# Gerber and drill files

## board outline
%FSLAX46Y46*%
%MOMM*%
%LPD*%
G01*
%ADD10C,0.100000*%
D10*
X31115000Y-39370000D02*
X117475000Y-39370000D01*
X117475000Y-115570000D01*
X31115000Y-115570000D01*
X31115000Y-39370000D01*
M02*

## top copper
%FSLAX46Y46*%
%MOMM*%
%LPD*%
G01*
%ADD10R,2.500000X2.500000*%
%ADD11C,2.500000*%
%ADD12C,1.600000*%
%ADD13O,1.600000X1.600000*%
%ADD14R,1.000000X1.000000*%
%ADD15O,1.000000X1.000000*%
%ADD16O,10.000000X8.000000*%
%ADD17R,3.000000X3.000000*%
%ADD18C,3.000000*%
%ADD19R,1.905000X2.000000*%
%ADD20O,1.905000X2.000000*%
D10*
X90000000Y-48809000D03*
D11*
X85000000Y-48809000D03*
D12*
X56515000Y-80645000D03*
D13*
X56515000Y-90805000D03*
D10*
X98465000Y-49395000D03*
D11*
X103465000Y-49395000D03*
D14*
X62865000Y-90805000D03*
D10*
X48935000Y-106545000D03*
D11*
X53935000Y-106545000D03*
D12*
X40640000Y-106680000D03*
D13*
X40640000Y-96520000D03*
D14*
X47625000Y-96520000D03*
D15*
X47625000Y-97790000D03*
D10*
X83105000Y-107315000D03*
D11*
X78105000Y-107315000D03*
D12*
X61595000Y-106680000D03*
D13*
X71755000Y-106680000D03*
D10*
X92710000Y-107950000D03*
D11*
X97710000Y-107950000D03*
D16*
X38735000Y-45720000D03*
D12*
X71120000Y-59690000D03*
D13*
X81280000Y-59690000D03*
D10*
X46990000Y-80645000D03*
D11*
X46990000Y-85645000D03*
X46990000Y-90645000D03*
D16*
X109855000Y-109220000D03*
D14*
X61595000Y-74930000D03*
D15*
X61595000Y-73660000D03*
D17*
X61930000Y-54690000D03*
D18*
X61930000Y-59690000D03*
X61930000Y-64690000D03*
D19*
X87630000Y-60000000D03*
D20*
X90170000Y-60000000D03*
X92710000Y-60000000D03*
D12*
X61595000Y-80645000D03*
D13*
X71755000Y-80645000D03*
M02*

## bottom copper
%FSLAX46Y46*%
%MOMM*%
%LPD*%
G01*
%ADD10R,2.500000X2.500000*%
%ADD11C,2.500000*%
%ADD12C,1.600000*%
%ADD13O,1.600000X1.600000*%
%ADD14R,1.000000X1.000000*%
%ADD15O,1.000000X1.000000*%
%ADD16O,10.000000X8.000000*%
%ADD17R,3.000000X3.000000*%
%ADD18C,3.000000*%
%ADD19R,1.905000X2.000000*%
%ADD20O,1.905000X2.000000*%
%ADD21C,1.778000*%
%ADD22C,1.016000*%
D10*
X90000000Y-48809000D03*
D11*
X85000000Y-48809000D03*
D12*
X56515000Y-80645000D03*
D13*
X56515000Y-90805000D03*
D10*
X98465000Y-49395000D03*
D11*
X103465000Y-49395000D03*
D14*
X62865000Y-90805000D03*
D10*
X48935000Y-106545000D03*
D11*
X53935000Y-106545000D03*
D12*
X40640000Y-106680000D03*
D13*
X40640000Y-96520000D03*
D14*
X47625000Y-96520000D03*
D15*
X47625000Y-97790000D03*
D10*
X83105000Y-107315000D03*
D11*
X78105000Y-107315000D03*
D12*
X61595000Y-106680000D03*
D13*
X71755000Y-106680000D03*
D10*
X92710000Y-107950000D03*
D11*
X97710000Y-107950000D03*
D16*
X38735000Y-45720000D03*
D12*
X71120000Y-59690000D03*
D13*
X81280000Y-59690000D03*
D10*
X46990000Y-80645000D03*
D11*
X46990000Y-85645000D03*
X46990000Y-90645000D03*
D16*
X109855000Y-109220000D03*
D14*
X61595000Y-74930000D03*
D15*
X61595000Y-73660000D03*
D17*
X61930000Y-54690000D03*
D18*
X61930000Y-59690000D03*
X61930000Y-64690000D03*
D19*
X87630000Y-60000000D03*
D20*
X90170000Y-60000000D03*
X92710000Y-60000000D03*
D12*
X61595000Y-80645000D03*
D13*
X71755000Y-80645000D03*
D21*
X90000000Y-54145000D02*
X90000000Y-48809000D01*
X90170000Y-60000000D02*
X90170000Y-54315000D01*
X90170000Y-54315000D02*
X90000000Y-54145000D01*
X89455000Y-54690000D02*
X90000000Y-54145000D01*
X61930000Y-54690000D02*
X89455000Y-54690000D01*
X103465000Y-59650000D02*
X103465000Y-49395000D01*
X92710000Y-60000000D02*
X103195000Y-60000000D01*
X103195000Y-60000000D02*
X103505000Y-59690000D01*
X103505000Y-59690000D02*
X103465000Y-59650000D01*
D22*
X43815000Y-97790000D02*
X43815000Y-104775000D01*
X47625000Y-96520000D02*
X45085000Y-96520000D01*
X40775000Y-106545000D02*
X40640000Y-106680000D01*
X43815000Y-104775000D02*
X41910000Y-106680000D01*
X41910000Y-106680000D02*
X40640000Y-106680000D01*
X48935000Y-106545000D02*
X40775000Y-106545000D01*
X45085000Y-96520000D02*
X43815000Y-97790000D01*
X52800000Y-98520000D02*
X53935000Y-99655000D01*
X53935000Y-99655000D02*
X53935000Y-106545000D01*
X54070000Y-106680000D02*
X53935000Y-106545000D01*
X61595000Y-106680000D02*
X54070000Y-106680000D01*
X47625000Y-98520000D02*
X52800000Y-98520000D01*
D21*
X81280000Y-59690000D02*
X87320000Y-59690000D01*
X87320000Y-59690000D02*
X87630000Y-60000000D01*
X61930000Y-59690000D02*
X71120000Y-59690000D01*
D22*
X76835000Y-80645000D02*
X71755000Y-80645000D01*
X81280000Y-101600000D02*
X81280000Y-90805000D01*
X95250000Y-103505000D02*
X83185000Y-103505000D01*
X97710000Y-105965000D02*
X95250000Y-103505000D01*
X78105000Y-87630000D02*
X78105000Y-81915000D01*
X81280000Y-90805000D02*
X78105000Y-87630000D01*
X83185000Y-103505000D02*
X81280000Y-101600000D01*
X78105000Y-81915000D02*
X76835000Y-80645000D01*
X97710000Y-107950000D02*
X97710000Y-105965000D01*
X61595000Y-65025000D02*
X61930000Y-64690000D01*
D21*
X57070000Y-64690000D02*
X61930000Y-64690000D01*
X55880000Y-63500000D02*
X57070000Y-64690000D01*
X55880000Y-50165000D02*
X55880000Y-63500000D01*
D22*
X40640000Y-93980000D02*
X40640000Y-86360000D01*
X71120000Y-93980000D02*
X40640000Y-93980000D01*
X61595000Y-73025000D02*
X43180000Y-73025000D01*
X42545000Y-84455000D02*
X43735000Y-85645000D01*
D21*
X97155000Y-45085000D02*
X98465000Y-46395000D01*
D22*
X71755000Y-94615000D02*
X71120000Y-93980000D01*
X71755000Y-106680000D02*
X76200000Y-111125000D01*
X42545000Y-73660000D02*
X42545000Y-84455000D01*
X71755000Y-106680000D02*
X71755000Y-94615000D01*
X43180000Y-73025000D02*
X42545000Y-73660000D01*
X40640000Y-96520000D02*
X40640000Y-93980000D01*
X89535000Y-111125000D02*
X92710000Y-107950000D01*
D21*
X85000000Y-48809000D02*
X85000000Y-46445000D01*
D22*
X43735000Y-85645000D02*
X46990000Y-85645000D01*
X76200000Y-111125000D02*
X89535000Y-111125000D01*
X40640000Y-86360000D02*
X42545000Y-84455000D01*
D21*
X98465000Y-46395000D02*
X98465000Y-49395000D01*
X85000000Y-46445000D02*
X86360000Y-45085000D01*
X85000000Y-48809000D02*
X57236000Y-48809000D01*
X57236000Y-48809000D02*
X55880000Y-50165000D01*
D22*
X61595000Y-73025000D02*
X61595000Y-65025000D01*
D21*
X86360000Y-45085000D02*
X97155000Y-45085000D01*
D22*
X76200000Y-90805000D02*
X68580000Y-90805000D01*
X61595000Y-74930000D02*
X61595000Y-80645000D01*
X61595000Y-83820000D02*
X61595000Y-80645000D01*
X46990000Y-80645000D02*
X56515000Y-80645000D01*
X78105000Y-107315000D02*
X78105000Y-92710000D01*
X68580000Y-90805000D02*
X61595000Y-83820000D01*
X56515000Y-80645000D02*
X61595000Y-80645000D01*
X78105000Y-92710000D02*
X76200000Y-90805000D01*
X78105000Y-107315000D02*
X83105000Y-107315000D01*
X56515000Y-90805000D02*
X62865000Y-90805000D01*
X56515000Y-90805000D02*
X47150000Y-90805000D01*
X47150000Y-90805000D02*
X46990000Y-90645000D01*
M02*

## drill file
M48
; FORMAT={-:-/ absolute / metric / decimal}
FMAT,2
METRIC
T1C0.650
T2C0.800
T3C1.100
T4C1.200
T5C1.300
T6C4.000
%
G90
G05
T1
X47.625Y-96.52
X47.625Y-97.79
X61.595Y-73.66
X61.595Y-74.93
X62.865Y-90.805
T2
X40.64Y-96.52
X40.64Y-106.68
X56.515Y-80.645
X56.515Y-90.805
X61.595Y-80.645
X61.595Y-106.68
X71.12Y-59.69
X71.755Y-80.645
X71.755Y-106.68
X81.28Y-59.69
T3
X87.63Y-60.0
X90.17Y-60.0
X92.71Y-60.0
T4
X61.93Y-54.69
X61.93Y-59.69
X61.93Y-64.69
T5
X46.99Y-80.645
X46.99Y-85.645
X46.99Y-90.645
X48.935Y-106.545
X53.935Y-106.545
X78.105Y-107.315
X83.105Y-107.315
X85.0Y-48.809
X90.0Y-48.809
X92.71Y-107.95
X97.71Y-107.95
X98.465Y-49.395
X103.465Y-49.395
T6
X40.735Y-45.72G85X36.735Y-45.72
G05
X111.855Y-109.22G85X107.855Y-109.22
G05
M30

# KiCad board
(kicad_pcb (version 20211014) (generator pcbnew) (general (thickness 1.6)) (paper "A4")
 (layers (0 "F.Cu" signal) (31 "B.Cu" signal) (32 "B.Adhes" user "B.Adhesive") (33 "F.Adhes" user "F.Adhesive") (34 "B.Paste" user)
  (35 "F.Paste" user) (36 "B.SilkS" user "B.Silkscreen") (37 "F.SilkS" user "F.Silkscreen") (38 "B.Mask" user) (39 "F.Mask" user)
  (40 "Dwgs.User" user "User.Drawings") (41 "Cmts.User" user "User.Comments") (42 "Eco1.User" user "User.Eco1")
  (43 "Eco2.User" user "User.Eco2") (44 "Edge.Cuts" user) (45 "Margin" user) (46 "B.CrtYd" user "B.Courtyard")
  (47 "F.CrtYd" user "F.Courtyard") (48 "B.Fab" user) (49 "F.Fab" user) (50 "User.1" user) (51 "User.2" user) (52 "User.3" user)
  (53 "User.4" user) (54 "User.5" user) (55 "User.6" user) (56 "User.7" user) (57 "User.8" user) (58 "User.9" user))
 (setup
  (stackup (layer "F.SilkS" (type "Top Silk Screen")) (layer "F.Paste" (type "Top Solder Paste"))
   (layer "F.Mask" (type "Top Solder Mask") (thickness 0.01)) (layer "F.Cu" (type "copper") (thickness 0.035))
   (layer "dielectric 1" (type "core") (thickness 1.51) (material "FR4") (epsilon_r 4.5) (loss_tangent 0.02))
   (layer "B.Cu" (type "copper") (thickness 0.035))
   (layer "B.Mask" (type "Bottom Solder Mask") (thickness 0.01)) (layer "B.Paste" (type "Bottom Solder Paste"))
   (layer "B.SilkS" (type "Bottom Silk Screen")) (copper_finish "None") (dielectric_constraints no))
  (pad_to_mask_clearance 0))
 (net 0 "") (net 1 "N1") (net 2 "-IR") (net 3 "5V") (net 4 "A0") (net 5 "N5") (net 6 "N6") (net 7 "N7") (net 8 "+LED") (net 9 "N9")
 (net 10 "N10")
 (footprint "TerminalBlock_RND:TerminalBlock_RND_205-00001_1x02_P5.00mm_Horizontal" (layer "F.Cu") (at 90 48.809 180)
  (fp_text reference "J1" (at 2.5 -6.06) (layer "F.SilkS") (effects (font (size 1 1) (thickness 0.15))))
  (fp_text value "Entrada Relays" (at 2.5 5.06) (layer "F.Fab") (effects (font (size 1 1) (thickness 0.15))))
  (pad "1" thru_hole rect (at 0 0 180) (size 2.5 2.5) (drill 1.3) (layers *.Cu *.Mask) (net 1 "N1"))
  (pad "2" thru_hole circle (at 5 0 180) (size 2.5 2.5) (drill 1.3) (layers *.Cu *.Mask) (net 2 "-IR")))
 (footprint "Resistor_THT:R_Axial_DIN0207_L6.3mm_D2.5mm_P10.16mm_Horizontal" (layer "F.Cu") (at 56.515 80.645 -90)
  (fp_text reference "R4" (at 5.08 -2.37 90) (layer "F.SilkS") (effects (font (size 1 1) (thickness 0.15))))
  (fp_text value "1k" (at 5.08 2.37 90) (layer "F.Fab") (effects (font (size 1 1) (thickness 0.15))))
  (pad "1" thru_hole circle (at 0 0 270) (size 1.6 1.6) (drill 0.8) (layers *.Cu *.Mask) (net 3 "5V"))
  (pad "2" thru_hole oval (at 10.16 0 270) (size 1.6 1.6) (drill 0.8) (layers *.Cu *.Mask) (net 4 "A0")))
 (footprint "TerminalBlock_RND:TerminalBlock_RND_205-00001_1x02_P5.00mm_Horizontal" (layer "F.Cu") (at 98.465 49.395)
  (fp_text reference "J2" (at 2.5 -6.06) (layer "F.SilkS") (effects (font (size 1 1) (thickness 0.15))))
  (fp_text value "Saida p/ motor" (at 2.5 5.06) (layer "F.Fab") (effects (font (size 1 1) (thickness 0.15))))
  (pad "1" thru_hole rect (at 0 0) (size 2.5 2.5) (drill 1.3) (layers *.Cu *.Mask) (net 2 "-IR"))
  (pad "2" thru_hole circle (at 5 0) (size 2.5 2.5) (drill 1.3) (layers *.Cu *.Mask) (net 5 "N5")))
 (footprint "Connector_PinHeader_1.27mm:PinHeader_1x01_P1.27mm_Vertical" (layer "F.Cu") (at 62.865 90.805)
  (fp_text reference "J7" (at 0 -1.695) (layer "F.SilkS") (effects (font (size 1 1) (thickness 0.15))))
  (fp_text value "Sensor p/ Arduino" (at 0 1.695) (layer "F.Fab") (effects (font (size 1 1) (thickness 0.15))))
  (pad "1" thru_hole rect (at 0 0) (size 1 1) (drill 0.65) (layers *.Cu *.Mask) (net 4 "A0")))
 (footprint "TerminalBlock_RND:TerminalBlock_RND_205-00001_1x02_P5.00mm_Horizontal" (layer "F.Cu") (at 48.935 106.545)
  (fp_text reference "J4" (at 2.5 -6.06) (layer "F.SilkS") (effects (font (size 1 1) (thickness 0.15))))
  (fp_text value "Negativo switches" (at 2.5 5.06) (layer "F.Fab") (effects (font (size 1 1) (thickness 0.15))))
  (pad "1" thru_hole rect (at 0 0) (size 2.5 2.5) (drill 1.3) (layers *.Cu *.Mask) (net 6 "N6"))
  (pad "2" thru_hole circle (at 5 0) (size 2.5 2.5) (drill 1.3) (layers *.Cu *.Mask) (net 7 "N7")))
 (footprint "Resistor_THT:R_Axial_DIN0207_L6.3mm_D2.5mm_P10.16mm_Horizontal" (layer "F.Cu") (at 40.64 106.68 90)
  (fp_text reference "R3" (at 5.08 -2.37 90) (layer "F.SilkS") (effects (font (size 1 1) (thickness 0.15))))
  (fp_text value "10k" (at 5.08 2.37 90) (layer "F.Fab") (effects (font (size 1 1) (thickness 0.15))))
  (pad "1" thru_hole circle (at 0 0 90) (size 1.6 1.6) (drill 0.8) (layers *.Cu *.Mask) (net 6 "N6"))
  (pad "2" thru_hole oval (at 10.16 0 90) (size 1.6 1.6) (drill 0.8) (layers *.Cu *.Mask) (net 2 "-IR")))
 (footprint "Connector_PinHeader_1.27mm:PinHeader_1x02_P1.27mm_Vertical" (layer "F.Cu") (at 47.625 96.52)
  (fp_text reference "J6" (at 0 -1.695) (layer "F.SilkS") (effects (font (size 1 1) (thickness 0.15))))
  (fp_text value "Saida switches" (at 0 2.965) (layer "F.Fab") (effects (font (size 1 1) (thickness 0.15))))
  (pad "1" thru_hole rect (at 0 0) (size 1 1) (drill 0.65) (layers *.Cu *.Mask) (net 6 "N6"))
  (pad "2" thru_hole oval (at 0 1.27) (size 1 1) (drill 0.65) (layers *.Cu *.Mask) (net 7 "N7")))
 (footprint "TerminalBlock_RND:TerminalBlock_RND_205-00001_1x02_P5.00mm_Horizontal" (layer "F.Cu") (at 83.105 107.315 180)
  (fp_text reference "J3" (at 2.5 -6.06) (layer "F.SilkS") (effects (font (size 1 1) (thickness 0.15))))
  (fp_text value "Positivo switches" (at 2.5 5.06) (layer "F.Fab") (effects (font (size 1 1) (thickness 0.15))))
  (pad "1" thru_hole rect (at 0 0 180) (size 2.5 2.5) (drill 1.3) (layers *.Cu *.Mask) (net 3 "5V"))
  (pad "2" thru_hole circle (at 5 0 180) (size 2.5 2.5) (drill 1.3) (layers *.Cu *.Mask) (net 3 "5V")))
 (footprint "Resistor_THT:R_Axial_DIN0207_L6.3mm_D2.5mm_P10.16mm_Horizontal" (layer "F.Cu") (at 61.595 106.68)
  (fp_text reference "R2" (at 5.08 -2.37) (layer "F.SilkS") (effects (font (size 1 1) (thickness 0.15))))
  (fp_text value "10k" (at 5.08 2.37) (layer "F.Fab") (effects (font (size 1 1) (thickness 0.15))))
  (pad "1" thru_hole circle (at 0 0) (size 1.6 1.6) (drill 0.8) (layers *.Cu *.Mask) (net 7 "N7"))
  (pad "2" thru_hole oval (at 10.16 0) (size 1.6 1.6) (drill 0.8) (layers *.Cu *.Mask) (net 2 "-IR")))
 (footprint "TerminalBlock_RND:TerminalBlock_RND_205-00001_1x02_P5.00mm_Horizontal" (layer "F.Cu") (at 92.71 107.95)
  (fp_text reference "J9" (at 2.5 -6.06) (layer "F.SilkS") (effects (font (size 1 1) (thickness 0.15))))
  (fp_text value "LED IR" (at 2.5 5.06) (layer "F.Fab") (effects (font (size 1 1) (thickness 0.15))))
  (pad "1" thru_hole rect (at 0 0) (size 2.5 2.5) (drill 1.3) (layers *.Cu *.Mask) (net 2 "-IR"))
  (pad "2" thru_hole circle (at 5 0) (size 2.5 2.5) (drill 1.3) (layers *.Cu *.Mask) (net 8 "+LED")))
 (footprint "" (layer "F.Cu") (at 38.735 45.72)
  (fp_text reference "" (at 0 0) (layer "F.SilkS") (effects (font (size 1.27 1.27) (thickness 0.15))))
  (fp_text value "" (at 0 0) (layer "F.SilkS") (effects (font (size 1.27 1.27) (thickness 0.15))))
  (pad "1" thru_hole oval (at 0 0 180) (size 10 8) (drill oval 8 4) (layers *.Cu *.Mask)))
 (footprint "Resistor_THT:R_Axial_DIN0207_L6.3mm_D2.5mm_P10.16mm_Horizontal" (layer "F.Cu") (at 71.12 59.69)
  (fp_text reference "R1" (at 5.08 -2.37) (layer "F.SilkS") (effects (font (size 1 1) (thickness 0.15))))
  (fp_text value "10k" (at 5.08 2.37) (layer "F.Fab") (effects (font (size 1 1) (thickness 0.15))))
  (pad "1" thru_hole circle (at 0 0) (size 1.6 1.6) (drill 0.8) (layers *.Cu *.Mask) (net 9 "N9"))
  (pad "2" thru_hole oval (at 10.16 0) (size 1.6 1.6) (drill 0.8) (layers *.Cu *.Mask) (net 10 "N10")))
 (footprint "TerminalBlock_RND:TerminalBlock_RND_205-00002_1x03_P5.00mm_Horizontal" (layer "F.Cu") (at 46.99 80.645 -90)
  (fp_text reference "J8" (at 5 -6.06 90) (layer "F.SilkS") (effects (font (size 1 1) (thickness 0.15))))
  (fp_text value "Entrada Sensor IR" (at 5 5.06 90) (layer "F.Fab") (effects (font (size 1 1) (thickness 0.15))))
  (pad "1" thru_hole rect (at 0 0 270) (size 2.5 2.5) (drill 1.3) (layers *.Cu *.Mask) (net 3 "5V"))
  (pad "2" thru_hole circle (at 5 0 270) (size 2.5 2.5) (drill 1.3) (layers *.Cu *.Mask) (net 2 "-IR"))
  (pad "3" thru_hole circle (at 10 0 270) (size 2.5 2.5) (drill 1.3) (layers *.Cu *.Mask) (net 4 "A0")))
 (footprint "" (layer "F.Cu") (at 109.855 109.22)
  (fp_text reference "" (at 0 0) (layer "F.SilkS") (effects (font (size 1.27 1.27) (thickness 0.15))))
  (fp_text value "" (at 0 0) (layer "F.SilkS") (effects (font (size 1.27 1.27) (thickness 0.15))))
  (pad "1" thru_hole oval (at 0 0 180) (size 10 8) (drill oval 8 4) (layers F&B.Cu *.Mask)))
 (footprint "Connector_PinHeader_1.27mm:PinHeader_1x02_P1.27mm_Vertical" (layer "F.Cu") (at 61.595 74.93 180)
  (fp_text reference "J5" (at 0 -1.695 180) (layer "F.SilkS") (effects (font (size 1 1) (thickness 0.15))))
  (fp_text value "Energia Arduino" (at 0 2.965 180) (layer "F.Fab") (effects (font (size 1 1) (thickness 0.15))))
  (pad "1" thru_hole rect (at 0 0 180) (size 1 1) (drill 0.65) (layers *.Cu *.Mask) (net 3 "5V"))
  (pad "2" thru_hole oval (at 0 1.27 180) (size 1 1) (drill 0.65) (layers *.Cu *.Mask) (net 2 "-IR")))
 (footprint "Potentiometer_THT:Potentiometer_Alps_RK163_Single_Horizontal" (layer "F.Cu") (at 61.93 54.69)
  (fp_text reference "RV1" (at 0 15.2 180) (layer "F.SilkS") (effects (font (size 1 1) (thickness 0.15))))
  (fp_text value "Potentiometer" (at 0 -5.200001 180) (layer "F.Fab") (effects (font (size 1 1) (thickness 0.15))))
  (pad "1" thru_hole rect (at 0 0 180) (size 3 3) (drill 1.2) (layers *.Cu *.Mask) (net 1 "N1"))
  (pad "2" thru_hole circle (at 0 5 180) (size 3 3) (drill 1.2) (layers *.Cu *.Mask) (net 9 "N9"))
  (pad "3" thru_hole circle (at 0 10 180) (size 3 3) (drill 1.2) (layers *.Cu *.Mask) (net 2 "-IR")))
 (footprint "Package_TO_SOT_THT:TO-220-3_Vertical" (layer "F.Cu") (at 87.63 60)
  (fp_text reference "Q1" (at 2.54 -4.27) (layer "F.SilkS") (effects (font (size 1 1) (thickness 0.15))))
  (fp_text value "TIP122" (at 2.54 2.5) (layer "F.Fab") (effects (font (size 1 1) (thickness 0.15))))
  (pad "1" thru_hole rect (at 0 0) (size 1.905 2) (drill 1.1) (layers *.Cu *.Mask) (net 10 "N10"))
  (pad "2" thru_hole oval (at 2.54 0) (size 1.905 2) (drill 1.1) (layers *.Cu *.Mask) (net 1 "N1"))
  (pad "3" thru_hole oval (at 5.08 0) (size 1.905 2) (drill 1.1) (layers *.Cu *.Mask) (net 5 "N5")))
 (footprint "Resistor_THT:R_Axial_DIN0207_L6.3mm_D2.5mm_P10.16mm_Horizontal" (layer "F.Cu") (at 61.595 80.645)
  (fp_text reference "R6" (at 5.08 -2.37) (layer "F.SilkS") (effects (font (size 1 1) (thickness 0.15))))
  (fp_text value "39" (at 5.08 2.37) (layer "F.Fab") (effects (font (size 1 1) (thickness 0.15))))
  (pad "1" thru_hole circle (at 0 0) (size 1.6 1.6) (drill 0.8) (layers *.Cu *.Mask) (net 3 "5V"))
  (pad "2" thru_hole oval (at 10.16 0) (size 1.6 1.6) (drill 0.8) (layers *.Cu *.Mask) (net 8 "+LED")))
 (gr_rect (start 117.475 39.37) (end 31.115 115.57) (layer "Edge.Cuts") (width 0.1) (fill none))
 (segment (start 90 54.145) (end 90 48.809) (width 1.778) (layer "B.Cu") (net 1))
 (segment (start 90.17 60) (end 90.17 54.315) (width 1.778) (layer "B.Cu") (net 1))
 (segment (start 90.17 54.315) (end 90 54.145) (width 1.778) (layer "B.Cu") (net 1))
 (segment (start 89.455 54.69) (end 90 54.145) (width 1.778) (layer "B.Cu") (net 1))
 (segment (start 61.93 54.69) (end 89.455 54.69) (width 1.778) (layer "B.Cu") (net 1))
 (segment (start 103.465 59.65) (end 103.465 49.395) (width 1.778) (layer "B.Cu") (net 5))
 (segment (start 92.71 60) (end 103.195 60) (width 1.778) (layer "B.Cu") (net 5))
 (segment (start 103.195 60) (end 103.505 59.69) (width 1.778) (layer "B.Cu") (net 5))
 (segment (start 103.505 59.69) (end 103.465 59.65) (width 1.778) (layer "B.Cu") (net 5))
 (segment (start 43.815 97.79) (end 43.815 104.775) (width 1.016) (layer "B.Cu") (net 6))
 (segment (start 47.625 96.52) (end 45.085 96.52) (width 1.016) (layer "B.Cu") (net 6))
 (segment (start 40.775 106.545) (end 40.64 106.68) (width 1.016) (layer "B.Cu") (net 6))
 (segment (start 43.815 104.775) (end 41.91 106.68) (width 1.016) (layer "B.Cu") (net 6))
 (segment (start 41.91 106.68) (end 40.64 106.68) (width 1.016) (layer "B.Cu") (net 6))
 (segment (start 48.935 106.545) (end 40.775 106.545) (width 1.016) (layer "B.Cu") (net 6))
 (segment (start 45.085 96.52) (end 43.815 97.79) (width 1.016) (layer "B.Cu") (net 6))
 (segment (start 52.8 98.52) (end 53.935 99.655) (width 1.016) (layer "B.Cu") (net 7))
 (segment (start 53.935 99.655) (end 53.935 106.545) (width 1.016) (layer "B.Cu") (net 7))
 (segment (start 54.07 106.68) (end 53.935 106.545) (width 1.016) (layer "B.Cu") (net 7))
 (segment (start 61.595 106.68) (end 54.07 106.68) (width 1.016) (layer "B.Cu") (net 7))
 (segment (start 47.625 98.52) (end 52.8 98.52) (width 1.016) (layer "B.Cu") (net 7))
 (segment (start 81.28 59.69) (end 87.32 59.69) (width 1.778) (layer "B.Cu") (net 10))
 (segment (start 87.32 59.69) (end 87.63 60) (width 1.778) (layer "B.Cu") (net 10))
 (segment (start 61.93 59.69) (end 71.12 59.69) (width 1.778) (layer "B.Cu") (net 9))
 (segment (start 76.835 80.645) (end 71.755 80.645) (width 1.016) (layer "B.Cu") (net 8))
 (segment (start 81.28 101.6) (end 81.28 90.805) (width 1.016) (layer "B.Cu") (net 8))
 (segment (start 95.25 103.505) (end 83.185 103.505) (width 1.016) (layer "B.Cu") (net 8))
 (segment (start 97.71 105.965) (end 95.25 103.505) (width 1.016) (layer "B.Cu") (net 8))
 (segment (start 78.105 87.63) (end 78.105 81.915) (width 1.016) (layer "B.Cu") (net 8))
 (segment (start 81.28 90.805) (end 78.105 87.63) (width 1.016) (layer "B.Cu") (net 8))
 (segment (start 83.185 103.505) (end 81.28 101.6) (width 1.016) (layer "B.Cu") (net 8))
 (segment (start 78.105 81.915) (end 76.835 80.645) (width 1.016) (layer "B.Cu") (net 8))
 (segment (start 97.71 107.95) (end 97.71 105.965) (width 1.016) (layer "B.Cu") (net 8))
 (segment (start 61.595 65.025) (end 61.93 64.69) (width 1.016) (layer "B.Cu") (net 2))
 (segment (start 57.07 64.69) (end 61.93 64.69) (width 1.778) (layer "B.Cu") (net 2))
 (segment (start 55.88 63.5) (end 57.07 64.69) (width 1.778) (layer "B.Cu") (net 2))
 (segment (start 55.88 50.165) (end 55.88 63.5) (width 1.778) (layer "B.Cu") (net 2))
 (segment (start 40.64 93.98) (end 40.64 86.36) (width 1.016) (layer "B.Cu") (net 2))
 (segment (start 71.12 93.98) (end 40.64 93.98) (width 1.016) (layer "B.Cu") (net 2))
 (segment (start 61.595 73.025) (end 43.18 73.025) (width 1.016) (layer "B.Cu") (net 2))
 (segment (start 42.545 84.455) (end 43.735 85.645) (width 1.016) (layer "B.Cu") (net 2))
 (segment (start 97.155 45.085) (end 98.465 46.395) (width 1.778) (layer "B.Cu") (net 2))
 (segment (start 71.755 94.615) (end 71.12 93.98) (width 1.016) (layer "B.Cu") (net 2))
 (segment (start 71.755 106.68) (end 76.2 111.125) (width 1.016) (layer "B.Cu") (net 2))
 (segment (start 42.545 73.66) (end 42.545 84.455) (width 1.016) (layer "B.Cu") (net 2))
 (segment (start 71.755 106.68) (end 71.755 94.615) (width 1.016) (layer "B.Cu") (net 2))
 (segment (start 43.18 73.025) (end 42.545 73.66) (width 1.016) (layer "B.Cu") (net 2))
 (segment (start 40.64 96.52) (end 40.64 93.98) (width 1.016) (layer "B.Cu") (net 2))
 (segment (start 89.535 111.125) (end 92.71 107.95) (width 1.016) (layer "B.Cu") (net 2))
 (segment (start 85 48.809) (end 85 46.445) (width 1.778) (layer "B.Cu") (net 2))
 (segment (start 43.735 85.645) (end 46.99 85.645) (width 1.016) (layer "B.Cu") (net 2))
 (segment (start 76.2 111.125) (end 89.535 111.125) (width 1.016) (layer "B.Cu") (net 2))
 (segment (start 40.64 86.36) (end 42.545 84.455) (width 1.016) (layer "B.Cu") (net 2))
 (segment (start 98.465 46.395) (end 98.465 49.395) (width 1.778) (layer "B.Cu") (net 2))
 (segment (start 85 46.445) (end 86.36 45.085) (width 1.778) (layer "B.Cu") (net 2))
 (segment (start 85 48.809) (end 57.236 48.809) (width 1.778) (layer "B.Cu") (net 2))
 (segment (start 57.236 48.809) (end 55.88 50.165) (width 1.778) (layer "B.Cu") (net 2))
 (segment (start 61.595 73.025) (end 61.595 65.025) (width 1.016) (layer "B.Cu") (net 2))
 (segment (start 86.36 45.085) (end 97.155 45.085) (width 1.778) (layer "B.Cu") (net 2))
 (segment (start 76.2 90.805) (end 68.58 90.805) (width 1.016) (layer "B.Cu") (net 3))
 (segment (start 61.595 74.93) (end 61.595 80.645) (width 1.016) (layer "B.Cu") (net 3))
 (segment (start 61.595 83.82) (end 61.595 80.645) (width 1.016) (layer "B.Cu") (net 3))
 (segment (start 46.99 80.645) (end 56.515 80.645) (width 1.016) (layer "B.Cu") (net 3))
 (segment (start 78.105 107.315) (end 78.105 92.71) (width 1.016) (layer "B.Cu") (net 3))
 (segment (start 68.58 90.805) (end 61.595 83.82) (width 1.016) (layer "B.Cu") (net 3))
 (segment (start 56.515 80.645) (end 61.595 80.645) (width 1.016) (layer "B.Cu") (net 3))
 (segment (start 78.105 92.71) (end 76.2 90.805) (width 1.016) (layer "B.Cu") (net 3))
 (segment (start 78.105 107.315) (end 83.105 107.315) (width 1.016) (layer "B.Cu") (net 3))
 (segment (start 56.515 90.805) (end 62.865 90.805) (width 1.016) (layer "B.Cu") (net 4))
 (segment (start 56.515 90.805) (end 47.15 90.805) (width 1.016) (layer "B.Cu") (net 4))
 (segment (start 47.15 90.805) (end 46.99 90.645) (width 1.016) (layer "B.Cu") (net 4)))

